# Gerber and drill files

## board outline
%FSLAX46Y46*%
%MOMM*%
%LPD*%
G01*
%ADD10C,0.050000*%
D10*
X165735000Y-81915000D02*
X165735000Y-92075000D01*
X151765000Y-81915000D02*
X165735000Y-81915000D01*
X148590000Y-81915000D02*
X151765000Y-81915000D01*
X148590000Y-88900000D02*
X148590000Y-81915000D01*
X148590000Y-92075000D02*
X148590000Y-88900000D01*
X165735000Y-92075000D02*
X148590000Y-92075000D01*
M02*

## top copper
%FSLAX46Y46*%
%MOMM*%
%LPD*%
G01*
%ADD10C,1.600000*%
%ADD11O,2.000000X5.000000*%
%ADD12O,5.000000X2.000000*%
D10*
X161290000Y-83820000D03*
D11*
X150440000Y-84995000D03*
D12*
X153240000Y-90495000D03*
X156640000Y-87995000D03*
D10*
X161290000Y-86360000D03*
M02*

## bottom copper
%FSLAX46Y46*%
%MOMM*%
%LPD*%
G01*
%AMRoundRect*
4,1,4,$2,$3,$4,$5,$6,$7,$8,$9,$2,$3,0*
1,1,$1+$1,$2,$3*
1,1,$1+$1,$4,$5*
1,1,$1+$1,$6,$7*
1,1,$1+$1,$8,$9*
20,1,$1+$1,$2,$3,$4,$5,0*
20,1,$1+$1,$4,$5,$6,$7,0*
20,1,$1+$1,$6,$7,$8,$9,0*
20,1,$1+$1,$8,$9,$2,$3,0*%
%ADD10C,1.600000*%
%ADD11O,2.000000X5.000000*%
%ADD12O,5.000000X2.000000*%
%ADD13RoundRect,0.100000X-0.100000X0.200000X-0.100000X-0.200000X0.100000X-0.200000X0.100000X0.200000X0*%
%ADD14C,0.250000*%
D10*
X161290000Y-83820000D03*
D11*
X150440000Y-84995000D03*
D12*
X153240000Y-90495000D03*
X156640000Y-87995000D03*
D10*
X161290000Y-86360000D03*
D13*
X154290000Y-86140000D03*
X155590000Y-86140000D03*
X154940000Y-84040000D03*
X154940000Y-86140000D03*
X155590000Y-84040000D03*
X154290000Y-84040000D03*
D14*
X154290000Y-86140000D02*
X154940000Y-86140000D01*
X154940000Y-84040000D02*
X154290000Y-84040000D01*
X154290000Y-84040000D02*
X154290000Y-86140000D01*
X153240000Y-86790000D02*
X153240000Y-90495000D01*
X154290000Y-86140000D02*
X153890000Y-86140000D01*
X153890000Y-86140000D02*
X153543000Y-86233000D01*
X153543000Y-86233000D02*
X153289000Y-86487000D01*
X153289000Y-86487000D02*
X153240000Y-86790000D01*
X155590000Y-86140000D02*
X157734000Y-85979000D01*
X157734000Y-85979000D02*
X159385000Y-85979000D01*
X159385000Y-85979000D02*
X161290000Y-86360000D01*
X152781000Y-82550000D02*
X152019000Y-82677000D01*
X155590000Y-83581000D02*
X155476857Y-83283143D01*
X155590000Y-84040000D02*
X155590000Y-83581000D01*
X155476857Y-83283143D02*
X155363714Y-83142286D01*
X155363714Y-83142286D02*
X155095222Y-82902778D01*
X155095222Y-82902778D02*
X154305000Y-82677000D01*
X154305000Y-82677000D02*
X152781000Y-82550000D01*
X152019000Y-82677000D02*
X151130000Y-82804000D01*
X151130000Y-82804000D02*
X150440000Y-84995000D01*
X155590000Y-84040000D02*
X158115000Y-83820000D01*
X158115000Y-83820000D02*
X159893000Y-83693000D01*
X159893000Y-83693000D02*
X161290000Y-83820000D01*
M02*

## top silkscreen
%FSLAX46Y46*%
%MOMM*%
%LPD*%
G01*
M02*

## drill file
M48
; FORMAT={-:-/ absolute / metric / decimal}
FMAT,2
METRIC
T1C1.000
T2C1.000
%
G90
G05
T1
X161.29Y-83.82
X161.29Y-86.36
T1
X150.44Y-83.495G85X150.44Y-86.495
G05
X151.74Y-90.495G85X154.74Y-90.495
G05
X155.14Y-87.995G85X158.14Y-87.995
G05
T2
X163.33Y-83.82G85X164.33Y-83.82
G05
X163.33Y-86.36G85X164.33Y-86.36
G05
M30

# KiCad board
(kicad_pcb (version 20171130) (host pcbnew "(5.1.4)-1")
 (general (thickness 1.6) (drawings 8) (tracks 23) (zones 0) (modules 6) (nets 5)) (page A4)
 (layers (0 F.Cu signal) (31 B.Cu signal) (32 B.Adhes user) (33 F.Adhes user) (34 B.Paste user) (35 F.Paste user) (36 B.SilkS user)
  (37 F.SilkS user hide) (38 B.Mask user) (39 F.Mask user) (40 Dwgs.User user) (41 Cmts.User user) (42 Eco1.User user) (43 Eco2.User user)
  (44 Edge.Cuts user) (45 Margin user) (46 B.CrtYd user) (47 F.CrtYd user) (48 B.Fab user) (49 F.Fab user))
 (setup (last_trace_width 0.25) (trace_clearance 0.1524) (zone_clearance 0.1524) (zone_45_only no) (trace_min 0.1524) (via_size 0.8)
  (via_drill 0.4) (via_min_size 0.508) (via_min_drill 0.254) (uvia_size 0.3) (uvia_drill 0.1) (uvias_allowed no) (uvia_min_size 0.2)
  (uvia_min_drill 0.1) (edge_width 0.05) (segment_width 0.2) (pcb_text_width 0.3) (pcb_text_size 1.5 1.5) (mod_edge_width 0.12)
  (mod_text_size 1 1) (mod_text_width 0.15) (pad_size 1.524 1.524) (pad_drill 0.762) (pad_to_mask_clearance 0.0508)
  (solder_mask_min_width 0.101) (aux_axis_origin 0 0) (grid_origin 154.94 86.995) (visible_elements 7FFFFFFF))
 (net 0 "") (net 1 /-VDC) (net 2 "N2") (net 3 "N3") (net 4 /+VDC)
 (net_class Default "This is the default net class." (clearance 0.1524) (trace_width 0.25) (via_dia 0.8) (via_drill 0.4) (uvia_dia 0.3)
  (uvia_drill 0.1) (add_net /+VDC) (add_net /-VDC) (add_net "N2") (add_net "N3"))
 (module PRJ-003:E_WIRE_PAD (layer F.Cu) (at 161.29 83.82)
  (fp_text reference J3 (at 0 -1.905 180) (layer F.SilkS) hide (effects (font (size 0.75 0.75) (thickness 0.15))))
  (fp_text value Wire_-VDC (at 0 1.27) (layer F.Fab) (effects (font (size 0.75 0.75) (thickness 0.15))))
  (pad "" connect circle (at 0 0) (size 1 1) (layers F.Mask))
  (pad 1 thru_hole circle (at 0 0) (size 1.6 1.6) (drill 1) (layers B.Cu B.Mask) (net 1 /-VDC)))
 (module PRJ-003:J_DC (layer F.Cu) (at 154.94 86.995)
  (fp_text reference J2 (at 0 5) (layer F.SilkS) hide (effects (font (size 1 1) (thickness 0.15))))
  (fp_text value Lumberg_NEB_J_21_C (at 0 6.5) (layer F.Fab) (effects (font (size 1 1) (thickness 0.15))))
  (pad "" connect oval (at -1.7 3.5 90) (size 1 4) (layers F.Mask))
  (pad "" connect oval (at 1.7 1 90) (size 1 4) (layers F.Mask))
  (pad "" connect oval (at -4.5 -2) (size 1 4) (layers F.Mask))
  (pad 1 thru_hole oval (at -4.5 -2) (size 2 5) (drill oval 1 4) (layers B.Cu B.Mask) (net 1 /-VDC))
  (pad 2 thru_hole oval (at -1.7 3.5) (size 5 2) (drill oval 4 1) (layers B.Cu B.Mask) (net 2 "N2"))
  (pad 3 thru_hole oval (at 1.7 1) (size 5 2) (drill oval 4 1) (layers B.Cu B.Mask) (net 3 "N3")))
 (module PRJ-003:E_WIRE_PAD (layer F.Cu) (at 161.29 86.36)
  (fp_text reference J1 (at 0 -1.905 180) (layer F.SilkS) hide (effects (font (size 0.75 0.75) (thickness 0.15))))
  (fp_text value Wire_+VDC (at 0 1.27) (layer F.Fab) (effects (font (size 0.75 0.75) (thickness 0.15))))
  (pad "" connect circle (at 0 0) (size 1 1) (layers F.Mask))
  (pad 1 thru_hole circle (at 0 0) (size 1.6 1.6) (drill 1) (layers B.Cu B.Mask) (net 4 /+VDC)))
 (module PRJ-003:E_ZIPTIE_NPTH (layer F.Cu) (at 163.83 86.36 90)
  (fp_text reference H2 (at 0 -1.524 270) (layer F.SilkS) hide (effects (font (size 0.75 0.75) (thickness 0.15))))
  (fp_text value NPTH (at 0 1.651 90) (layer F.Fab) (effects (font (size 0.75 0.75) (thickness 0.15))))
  (pad "" np_thru_hole oval (at 0 0 90) (size 1 2) (drill oval 1 2) (layers *.Cu *.Mask)))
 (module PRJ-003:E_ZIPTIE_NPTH (layer F.Cu) (at 163.83 83.82 90)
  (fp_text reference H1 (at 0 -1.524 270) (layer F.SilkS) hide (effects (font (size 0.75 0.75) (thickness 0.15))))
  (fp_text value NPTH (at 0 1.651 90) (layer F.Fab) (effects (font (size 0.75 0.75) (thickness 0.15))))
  (pad "" np_thru_hole oval (at 0 0 90) (size 1 2) (drill oval 1 2) (layers *.Cu *.Mask)))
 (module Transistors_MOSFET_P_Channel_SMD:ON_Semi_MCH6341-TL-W (layer B.Cu) (at 154.94 85.09 270)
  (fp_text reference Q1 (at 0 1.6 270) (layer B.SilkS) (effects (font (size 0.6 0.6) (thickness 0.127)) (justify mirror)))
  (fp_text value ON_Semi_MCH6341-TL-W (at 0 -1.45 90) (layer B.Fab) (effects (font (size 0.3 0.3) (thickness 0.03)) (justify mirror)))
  (pad 6 smd roundrect (at 1.05 0.65 270) (size 0.6 0.4) (layers B.Cu B.Paste B.Mask) (roundrect_rratio 0.25) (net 2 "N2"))
  (pad 4 smd roundrect (at 1.05 -0.65 270) (size 0.6 0.4) (layers B.Cu B.Paste B.Mask) (roundrect_rratio 0.25) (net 4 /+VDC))
  (pad 2 smd roundrect (at -1.05 0 270) (size 0.6 0.4) (layers B.Cu B.Paste B.Mask) (roundrect_rratio 0.25) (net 2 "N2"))
  (pad 5 smd roundrect (at 1.05 0 270) (size 0.6 0.4) (layers B.Cu B.Paste B.Mask) (roundrect_rratio 0.25) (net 2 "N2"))
  (pad 3 smd roundrect (at -1.05 -0.65 270) (size 0.6 0.4) (layers B.Cu B.Paste B.Mask) (roundrect_rratio 0.25) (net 1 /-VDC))
  (pad 1 smd roundrect (at -1.05 0.65 270) (size 0.6 0.4) (layers B.Cu B.Paste B.Mask) (roundrect_rratio 0.25) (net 2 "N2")))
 (gr_line (start 165.735 81.915) (end 165.735 92.075) (layer Edge.Cuts) (width 0.05))
 (gr_line (start 151.765 81.915) (end 165.735 81.915) (layer Edge.Cuts) (width 0.05))
 (gr_line (start 148.59 81.915) (end 151.765 81.915) (layer Edge.Cuts) (width 0.05))
 (gr_line (start 148.59 88.9) (end 148.59 81.915) (layer Edge.Cuts) (width 0.05))
 (gr_line (start 148.59 92.075) (end 148.59 88.9) (layer Edge.Cuts) (width 0.05))
 (gr_line (start 165.735 92.075) (end 148.59 92.075) (layer Edge.Cuts) (width 0.05))
 (segment (start 154.29 86.14) (end 154.94 86.14) (width 0.25) (layer B.Cu) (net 2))
 (segment (start 154.94 84.04) (end 154.29 84.04) (width 0.25) (layer B.Cu) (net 2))
 (segment (start 154.29 84.04) (end 154.29 86.14) (width 0.25) (layer B.Cu) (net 2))
 (segment (start 153.24 86.79) (end 153.24 90.495) (width 0.25) (layer B.Cu) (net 2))
 (segment (start 154.29 86.14) (end 153.89 86.14) (width 0.25) (layer B.Cu) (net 2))
 (segment (start 153.89 86.14) (end 153.543 86.233) (width 0.25) (layer B.Cu) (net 2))
 (segment (start 153.543 86.233) (end 153.289 86.487) (width 0.25) (layer B.Cu) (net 2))
 (segment (start 153.289 86.487) (end 153.24 86.79) (width 0.25) (layer B.Cu) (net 2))
 (segment (start 155.59 86.14) (end 157.734 85.979) (width 0.25) (layer B.Cu) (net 4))
 (segment (start 157.734 85.979) (end 159.385 85.979) (width 0.25) (layer B.Cu) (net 4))
 (segment (start 159.385 85.979) (end 161.29 86.36) (width 0.25) (layer B.Cu) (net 4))
 (segment (start 152.781 82.55) (end 152.019 82.677) (width 0.25) (layer B.Cu) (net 1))
 (segment (start 155.59 83.581) (end 155.476857 83.283143) (width 0.25) (layer B.Cu) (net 1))
 (segment (start 155.59 84.04) (end 155.59 83.581) (width 0.25) (layer B.Cu) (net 1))
 (segment (start 155.476857 83.283143) (end 155.363714 83.142286) (width 0.25) (layer B.Cu) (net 1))
 (segment (start 155.363714 83.142286) (end 155.095222 82.902778) (width 0.25) (layer B.Cu) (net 1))
 (segment (start 155.095222 82.902778) (end 154.305 82.677) (width 0.25) (layer B.Cu) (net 1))
 (segment (start 154.305 82.677) (end 152.781 82.55) (width 0.25) (layer B.Cu) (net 1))
 (segment (start 152.019 82.677) (end 151.13 82.804) (width 0.25) (layer B.Cu) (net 1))
 (segment (start 151.13 82.804) (end 150.44 84.995) (width 0.25) (layer B.Cu) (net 1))
 (segment (start 155.59 84.04) (end 158.115 83.82) (width 0.25) (layer B.Cu) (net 1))
 (segment (start 158.115 83.82) (end 159.893 83.693) (width 0.25) (layer B.Cu) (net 1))
 (segment (start 159.893 83.693) (end 161.29 83.82) (width 0.25) (layer B.Cu) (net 1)))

